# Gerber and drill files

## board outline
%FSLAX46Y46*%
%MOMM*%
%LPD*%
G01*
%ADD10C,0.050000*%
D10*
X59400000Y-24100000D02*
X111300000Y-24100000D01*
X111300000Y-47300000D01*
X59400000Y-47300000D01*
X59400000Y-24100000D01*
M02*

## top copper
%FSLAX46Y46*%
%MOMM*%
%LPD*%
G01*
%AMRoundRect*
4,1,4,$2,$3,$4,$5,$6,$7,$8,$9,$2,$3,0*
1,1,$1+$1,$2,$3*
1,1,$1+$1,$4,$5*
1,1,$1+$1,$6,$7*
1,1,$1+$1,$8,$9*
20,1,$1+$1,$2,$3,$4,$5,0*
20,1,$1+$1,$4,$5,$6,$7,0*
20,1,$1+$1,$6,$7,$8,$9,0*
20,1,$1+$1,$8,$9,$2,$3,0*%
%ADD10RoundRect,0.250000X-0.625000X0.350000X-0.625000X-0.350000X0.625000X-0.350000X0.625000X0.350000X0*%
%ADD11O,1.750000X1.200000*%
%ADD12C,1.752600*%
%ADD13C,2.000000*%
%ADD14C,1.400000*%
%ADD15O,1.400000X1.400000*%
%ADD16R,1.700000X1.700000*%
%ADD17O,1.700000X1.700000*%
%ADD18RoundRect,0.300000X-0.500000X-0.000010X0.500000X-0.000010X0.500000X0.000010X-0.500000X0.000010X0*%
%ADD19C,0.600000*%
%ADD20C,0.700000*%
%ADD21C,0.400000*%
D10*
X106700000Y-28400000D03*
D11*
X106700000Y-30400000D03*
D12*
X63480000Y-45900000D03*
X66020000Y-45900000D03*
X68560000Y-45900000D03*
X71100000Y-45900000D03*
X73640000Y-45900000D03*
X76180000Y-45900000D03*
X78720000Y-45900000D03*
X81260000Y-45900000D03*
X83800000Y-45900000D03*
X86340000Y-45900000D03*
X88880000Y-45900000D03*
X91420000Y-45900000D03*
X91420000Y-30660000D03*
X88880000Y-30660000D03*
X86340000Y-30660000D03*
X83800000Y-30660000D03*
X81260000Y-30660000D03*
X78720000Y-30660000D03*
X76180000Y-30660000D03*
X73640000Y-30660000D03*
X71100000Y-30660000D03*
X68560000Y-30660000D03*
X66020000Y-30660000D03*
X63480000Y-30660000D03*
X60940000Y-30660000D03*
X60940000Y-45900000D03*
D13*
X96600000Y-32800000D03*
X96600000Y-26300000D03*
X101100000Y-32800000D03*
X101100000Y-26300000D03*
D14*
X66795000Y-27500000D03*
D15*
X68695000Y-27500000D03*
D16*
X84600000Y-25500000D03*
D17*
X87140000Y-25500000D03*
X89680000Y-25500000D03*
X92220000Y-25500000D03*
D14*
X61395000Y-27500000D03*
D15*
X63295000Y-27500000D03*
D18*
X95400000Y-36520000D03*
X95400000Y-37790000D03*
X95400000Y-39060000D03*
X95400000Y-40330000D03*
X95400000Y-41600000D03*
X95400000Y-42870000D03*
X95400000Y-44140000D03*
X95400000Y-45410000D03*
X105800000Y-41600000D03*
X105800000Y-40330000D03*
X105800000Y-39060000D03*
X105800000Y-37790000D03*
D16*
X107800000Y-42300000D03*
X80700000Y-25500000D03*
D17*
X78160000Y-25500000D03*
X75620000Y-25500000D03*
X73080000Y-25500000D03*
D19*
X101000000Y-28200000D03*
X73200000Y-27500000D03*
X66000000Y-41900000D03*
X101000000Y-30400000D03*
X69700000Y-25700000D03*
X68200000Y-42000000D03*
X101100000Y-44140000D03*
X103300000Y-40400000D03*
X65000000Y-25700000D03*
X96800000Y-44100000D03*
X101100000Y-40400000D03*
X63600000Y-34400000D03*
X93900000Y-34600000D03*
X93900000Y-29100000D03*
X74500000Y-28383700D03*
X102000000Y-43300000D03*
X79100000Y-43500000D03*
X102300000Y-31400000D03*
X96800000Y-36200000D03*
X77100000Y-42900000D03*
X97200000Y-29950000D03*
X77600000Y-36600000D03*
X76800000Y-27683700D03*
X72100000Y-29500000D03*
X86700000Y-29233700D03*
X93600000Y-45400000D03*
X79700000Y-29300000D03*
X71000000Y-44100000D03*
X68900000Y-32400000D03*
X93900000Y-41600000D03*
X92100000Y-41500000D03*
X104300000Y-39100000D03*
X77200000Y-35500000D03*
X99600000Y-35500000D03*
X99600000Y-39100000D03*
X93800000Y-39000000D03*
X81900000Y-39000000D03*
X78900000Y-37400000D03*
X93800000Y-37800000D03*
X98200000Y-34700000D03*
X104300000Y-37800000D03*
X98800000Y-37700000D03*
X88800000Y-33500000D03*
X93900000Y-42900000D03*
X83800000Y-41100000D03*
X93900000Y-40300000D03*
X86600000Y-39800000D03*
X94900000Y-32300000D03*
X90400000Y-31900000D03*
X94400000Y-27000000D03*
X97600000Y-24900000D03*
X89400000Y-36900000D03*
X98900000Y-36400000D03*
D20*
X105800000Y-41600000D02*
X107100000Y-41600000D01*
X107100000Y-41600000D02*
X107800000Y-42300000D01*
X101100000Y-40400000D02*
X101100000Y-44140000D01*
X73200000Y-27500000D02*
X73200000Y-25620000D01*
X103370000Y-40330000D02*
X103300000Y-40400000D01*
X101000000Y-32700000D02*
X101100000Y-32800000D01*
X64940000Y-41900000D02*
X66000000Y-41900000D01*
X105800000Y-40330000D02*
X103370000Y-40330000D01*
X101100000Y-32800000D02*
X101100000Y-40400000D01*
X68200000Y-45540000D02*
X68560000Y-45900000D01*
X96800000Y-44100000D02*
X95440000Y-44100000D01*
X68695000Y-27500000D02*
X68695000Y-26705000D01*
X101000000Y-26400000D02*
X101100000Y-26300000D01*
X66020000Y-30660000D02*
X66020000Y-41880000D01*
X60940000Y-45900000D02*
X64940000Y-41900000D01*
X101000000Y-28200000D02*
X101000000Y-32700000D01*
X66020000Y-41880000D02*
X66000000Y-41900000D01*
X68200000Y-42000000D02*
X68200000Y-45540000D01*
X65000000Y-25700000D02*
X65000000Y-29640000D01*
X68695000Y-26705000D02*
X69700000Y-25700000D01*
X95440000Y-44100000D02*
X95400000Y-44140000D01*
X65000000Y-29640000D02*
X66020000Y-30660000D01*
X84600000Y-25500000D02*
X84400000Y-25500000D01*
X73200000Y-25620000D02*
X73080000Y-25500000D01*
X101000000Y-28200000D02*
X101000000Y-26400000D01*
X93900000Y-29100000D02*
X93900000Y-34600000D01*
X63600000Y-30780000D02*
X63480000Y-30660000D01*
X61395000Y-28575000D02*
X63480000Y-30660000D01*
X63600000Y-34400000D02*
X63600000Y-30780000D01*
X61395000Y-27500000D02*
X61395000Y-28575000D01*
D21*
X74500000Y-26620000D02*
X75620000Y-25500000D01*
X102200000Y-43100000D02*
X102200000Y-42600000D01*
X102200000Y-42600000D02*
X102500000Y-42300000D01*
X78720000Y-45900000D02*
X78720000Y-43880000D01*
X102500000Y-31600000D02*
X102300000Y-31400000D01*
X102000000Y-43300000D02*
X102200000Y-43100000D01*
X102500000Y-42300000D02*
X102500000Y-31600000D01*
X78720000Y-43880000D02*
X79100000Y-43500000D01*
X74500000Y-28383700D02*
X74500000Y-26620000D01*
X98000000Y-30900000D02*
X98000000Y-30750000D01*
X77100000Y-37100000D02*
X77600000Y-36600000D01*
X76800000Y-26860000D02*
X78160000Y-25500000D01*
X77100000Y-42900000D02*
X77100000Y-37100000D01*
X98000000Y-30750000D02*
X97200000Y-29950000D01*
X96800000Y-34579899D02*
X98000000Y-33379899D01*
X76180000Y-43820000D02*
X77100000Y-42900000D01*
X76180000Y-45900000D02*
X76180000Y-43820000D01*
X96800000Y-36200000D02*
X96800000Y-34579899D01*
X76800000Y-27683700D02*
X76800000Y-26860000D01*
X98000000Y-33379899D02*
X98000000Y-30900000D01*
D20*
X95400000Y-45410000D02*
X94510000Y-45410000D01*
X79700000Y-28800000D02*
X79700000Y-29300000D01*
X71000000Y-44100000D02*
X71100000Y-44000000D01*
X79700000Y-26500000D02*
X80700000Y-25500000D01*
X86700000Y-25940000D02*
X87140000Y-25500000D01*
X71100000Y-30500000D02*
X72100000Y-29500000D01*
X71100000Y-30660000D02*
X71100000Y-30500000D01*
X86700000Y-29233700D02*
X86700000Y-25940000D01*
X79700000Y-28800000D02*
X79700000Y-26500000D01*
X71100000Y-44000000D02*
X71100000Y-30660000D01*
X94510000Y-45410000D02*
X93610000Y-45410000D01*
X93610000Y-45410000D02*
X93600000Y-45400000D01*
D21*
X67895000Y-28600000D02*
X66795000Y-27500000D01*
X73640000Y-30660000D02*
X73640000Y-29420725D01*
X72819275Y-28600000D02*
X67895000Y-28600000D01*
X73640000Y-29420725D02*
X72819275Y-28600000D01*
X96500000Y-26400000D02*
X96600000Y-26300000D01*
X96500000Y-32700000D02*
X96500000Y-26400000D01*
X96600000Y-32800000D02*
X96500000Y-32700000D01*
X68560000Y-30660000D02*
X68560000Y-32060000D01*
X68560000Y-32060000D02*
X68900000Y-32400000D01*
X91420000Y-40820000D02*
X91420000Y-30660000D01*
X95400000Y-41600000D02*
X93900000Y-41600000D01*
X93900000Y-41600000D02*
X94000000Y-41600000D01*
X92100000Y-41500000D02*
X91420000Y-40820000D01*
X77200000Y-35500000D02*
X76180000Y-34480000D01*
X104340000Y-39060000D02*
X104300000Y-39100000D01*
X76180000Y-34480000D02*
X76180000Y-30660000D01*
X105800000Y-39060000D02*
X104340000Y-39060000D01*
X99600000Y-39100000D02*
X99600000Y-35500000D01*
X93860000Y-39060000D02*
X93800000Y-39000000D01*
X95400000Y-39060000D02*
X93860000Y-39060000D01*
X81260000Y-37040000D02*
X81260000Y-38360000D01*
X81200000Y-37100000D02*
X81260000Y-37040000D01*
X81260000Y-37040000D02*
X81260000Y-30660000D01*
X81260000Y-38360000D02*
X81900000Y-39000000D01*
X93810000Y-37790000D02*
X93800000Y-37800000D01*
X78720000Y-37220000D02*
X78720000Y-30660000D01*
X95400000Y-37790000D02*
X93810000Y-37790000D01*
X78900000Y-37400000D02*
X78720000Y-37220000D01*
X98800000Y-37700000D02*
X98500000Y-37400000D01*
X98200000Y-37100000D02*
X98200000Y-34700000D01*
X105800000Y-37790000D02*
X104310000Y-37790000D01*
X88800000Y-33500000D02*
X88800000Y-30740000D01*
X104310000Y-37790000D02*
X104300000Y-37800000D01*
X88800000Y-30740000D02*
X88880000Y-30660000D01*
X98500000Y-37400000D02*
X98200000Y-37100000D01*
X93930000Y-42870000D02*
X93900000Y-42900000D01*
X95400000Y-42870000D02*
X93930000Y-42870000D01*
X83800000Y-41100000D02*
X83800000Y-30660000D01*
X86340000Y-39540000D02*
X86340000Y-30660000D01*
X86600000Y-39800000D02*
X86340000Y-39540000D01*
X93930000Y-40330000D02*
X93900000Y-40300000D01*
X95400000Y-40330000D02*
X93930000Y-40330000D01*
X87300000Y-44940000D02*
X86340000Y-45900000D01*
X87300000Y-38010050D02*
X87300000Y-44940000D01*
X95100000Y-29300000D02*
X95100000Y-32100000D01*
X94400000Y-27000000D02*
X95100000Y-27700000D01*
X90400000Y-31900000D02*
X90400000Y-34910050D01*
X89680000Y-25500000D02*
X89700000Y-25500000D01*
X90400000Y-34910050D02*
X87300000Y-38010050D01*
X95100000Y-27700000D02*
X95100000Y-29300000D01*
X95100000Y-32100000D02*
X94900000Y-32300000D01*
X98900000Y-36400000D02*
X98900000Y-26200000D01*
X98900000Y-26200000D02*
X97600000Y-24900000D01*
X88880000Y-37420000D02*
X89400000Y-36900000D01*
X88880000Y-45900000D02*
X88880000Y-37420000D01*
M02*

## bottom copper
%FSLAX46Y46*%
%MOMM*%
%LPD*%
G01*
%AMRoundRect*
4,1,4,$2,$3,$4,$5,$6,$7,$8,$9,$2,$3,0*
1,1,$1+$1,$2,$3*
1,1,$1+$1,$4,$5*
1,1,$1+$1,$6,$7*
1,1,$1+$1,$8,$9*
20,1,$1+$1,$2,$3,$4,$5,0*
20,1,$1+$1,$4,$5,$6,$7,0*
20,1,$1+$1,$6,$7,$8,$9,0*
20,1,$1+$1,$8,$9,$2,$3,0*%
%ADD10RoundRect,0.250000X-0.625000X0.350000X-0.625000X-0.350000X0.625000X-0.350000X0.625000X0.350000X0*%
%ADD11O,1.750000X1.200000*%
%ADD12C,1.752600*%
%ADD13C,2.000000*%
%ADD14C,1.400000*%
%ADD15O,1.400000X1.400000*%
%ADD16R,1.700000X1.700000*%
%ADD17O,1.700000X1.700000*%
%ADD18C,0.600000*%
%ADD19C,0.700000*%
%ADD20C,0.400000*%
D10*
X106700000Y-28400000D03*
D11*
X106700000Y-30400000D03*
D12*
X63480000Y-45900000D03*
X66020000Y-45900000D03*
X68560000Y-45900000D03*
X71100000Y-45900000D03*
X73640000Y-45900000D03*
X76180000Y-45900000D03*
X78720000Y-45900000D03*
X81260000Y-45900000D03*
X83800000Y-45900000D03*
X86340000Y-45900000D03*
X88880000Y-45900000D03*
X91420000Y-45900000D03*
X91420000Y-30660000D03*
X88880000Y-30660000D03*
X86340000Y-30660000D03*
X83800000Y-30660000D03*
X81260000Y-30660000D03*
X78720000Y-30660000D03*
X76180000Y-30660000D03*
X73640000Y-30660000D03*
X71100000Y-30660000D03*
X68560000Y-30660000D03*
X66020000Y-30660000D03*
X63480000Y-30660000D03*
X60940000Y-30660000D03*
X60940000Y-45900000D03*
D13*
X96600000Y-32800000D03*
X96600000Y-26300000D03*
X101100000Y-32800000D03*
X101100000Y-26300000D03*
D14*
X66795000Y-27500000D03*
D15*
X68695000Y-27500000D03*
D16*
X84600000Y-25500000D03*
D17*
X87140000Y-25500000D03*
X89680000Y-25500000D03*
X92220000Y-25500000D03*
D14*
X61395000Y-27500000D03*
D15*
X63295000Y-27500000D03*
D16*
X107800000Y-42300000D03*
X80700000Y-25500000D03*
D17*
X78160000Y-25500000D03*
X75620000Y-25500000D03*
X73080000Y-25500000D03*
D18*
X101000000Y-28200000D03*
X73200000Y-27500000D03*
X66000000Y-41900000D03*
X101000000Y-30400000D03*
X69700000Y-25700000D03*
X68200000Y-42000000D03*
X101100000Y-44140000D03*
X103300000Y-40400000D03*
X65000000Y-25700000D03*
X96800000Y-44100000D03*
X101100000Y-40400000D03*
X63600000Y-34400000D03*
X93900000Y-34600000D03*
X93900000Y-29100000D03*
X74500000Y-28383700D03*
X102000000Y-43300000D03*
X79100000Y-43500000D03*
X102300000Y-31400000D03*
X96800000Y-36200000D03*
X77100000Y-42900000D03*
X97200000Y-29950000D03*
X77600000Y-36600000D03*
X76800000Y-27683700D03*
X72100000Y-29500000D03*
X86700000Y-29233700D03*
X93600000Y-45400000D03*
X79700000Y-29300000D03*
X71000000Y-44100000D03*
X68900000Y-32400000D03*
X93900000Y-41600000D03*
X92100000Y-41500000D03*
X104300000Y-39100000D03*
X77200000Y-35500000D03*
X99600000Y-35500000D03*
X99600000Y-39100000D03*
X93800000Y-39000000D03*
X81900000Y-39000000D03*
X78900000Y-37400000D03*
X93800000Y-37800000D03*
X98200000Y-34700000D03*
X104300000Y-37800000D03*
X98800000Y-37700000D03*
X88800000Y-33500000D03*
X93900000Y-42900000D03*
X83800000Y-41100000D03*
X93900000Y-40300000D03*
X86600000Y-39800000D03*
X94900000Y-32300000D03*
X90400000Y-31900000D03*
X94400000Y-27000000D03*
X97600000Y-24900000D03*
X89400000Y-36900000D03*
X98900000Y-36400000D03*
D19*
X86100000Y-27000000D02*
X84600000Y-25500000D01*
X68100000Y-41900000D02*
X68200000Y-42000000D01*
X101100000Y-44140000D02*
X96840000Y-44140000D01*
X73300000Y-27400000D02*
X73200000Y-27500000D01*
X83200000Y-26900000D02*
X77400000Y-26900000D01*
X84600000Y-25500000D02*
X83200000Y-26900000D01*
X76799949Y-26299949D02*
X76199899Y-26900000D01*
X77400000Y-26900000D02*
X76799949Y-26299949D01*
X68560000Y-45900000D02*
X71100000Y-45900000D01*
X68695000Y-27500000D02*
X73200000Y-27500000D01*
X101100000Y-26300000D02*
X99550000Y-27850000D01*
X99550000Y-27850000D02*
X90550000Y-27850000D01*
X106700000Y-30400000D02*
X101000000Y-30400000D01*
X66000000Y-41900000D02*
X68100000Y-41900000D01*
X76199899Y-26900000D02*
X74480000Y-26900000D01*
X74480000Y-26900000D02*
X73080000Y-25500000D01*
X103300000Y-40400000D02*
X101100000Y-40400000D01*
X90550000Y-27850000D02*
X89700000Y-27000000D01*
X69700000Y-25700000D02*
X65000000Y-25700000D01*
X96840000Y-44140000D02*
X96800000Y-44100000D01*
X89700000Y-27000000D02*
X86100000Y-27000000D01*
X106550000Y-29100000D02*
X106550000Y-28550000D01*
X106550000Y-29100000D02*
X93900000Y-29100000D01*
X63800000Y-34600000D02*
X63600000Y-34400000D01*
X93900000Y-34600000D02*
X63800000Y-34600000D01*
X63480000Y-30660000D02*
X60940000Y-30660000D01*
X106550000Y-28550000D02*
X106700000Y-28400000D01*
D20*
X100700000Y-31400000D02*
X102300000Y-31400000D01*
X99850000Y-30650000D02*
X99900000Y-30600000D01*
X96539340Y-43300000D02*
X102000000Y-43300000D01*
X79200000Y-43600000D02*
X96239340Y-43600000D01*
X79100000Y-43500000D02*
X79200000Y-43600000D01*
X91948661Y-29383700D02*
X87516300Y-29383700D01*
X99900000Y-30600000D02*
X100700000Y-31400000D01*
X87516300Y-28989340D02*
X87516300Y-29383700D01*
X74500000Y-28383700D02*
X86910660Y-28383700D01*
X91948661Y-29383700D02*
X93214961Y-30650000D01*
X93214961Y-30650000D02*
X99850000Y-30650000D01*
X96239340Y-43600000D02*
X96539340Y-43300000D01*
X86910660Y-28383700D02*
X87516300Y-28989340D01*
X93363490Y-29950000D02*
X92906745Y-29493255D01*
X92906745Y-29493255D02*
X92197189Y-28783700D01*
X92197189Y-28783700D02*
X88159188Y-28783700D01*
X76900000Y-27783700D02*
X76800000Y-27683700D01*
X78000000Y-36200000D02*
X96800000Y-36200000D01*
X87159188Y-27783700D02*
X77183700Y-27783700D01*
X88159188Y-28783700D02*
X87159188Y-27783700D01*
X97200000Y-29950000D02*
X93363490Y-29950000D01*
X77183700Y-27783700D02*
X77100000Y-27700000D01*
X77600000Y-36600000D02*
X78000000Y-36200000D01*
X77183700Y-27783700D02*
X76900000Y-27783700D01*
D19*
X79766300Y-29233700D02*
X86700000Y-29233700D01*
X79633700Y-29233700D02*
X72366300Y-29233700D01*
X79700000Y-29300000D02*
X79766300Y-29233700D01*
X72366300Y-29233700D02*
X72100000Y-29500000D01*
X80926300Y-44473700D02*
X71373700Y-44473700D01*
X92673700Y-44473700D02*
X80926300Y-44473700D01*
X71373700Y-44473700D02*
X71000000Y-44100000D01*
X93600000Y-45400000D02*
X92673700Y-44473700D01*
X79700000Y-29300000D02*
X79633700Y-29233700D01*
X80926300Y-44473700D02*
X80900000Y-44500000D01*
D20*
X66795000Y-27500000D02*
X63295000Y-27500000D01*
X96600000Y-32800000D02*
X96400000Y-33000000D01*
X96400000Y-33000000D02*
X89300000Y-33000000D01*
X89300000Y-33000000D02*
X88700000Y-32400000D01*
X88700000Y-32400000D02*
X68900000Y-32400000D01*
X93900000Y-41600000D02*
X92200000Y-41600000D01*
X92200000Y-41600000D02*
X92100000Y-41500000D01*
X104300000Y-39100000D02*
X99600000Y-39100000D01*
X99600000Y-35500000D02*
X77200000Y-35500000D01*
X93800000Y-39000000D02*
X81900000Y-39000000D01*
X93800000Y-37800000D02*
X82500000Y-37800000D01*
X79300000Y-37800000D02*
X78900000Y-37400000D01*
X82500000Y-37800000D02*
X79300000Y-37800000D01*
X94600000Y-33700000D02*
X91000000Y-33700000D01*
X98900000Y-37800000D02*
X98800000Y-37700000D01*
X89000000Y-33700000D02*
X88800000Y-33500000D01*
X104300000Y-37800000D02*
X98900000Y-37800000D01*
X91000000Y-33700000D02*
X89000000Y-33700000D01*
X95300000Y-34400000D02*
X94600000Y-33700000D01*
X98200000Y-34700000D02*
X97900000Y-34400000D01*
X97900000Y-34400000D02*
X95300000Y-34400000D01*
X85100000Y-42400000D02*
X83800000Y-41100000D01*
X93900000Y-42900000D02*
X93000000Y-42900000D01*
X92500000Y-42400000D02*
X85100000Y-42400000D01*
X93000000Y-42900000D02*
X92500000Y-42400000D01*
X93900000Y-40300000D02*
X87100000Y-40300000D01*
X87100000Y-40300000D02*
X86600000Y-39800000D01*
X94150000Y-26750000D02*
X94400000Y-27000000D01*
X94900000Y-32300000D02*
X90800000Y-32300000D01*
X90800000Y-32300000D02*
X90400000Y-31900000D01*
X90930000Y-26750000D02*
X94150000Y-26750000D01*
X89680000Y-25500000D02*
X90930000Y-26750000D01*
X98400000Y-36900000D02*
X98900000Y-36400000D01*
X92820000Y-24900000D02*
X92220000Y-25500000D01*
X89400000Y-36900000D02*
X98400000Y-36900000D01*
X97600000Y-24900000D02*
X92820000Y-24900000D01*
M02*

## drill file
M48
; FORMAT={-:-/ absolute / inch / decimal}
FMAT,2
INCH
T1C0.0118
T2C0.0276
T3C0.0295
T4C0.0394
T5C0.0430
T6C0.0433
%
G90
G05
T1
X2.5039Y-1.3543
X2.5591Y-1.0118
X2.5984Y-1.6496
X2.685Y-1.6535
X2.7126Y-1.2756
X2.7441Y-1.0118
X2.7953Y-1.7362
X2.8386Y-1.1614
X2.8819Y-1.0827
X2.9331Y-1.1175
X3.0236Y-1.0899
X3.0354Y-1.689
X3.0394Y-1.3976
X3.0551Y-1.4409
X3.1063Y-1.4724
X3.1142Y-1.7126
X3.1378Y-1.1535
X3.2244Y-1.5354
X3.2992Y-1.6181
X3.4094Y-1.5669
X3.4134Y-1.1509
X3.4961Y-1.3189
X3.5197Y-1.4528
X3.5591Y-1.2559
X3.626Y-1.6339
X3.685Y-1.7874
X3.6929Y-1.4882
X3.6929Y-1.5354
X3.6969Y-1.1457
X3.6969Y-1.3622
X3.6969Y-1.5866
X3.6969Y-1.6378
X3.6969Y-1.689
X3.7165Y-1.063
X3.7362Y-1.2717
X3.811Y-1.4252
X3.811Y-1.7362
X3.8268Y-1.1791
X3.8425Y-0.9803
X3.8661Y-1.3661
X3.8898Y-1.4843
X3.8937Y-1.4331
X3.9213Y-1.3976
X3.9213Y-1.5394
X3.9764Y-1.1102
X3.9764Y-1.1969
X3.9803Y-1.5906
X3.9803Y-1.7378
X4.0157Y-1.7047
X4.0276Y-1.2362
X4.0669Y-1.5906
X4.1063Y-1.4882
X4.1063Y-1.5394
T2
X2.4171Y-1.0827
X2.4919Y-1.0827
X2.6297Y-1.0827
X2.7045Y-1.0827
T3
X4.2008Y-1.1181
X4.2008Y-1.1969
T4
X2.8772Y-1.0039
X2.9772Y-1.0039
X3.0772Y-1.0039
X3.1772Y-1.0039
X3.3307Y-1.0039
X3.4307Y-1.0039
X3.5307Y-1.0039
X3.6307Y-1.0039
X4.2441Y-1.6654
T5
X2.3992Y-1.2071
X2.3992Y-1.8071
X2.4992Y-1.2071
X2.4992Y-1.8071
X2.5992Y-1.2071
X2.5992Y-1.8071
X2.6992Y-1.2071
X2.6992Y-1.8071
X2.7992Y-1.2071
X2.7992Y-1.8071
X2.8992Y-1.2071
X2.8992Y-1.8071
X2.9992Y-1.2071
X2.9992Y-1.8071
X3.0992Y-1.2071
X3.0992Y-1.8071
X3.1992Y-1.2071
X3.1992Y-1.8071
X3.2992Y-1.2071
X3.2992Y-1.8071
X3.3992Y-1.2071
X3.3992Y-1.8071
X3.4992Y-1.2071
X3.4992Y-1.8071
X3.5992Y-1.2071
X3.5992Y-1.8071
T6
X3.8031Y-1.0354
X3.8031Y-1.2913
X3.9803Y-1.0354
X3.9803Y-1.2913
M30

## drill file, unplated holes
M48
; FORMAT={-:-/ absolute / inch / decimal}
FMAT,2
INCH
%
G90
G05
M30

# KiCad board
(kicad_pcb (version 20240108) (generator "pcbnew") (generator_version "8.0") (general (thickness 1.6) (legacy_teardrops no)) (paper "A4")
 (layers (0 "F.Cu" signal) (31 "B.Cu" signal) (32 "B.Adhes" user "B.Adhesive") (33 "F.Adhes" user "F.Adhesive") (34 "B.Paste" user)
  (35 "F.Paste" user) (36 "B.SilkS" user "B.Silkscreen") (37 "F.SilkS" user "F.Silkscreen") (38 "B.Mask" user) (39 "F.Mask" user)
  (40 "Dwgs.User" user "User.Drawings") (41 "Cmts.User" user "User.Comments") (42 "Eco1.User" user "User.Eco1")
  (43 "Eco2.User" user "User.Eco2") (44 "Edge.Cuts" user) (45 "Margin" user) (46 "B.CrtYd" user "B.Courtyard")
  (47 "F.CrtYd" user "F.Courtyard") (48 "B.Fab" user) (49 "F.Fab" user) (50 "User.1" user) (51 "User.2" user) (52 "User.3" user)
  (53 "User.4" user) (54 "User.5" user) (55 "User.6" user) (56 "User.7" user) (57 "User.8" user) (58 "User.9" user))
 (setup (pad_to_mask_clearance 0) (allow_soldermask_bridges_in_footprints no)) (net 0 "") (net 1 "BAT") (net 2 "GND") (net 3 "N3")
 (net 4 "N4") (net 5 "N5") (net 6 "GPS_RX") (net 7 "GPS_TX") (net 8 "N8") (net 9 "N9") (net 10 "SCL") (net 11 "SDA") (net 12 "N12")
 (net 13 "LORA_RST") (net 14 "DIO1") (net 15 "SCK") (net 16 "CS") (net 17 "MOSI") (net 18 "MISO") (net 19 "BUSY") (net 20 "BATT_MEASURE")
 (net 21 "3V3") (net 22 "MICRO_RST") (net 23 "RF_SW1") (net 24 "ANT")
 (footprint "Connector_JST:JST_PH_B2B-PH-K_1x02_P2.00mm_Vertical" (layer "F.Cu") (at 106.7 28.4 -90)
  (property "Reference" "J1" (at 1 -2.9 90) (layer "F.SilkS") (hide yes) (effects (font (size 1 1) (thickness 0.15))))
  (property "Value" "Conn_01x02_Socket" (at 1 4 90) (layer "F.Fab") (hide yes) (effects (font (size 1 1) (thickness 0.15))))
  (pad "1" thru_hole roundrect (at 0 0 270) (size 1.2 1.75) (drill 0.75) (layers "*.Cu" "*.Mask") (remove_unused_layers no)
   (roundrect_rratio 0.208333) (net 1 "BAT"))
  (pad "2" thru_hole oval (at 2 0 270) (size 1.2 1.75) (drill 0.75) (layers "*.Cu" "*.Mask") (remove_unused_layers no) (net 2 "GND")))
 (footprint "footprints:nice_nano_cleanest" (layer "F.Cu") (at 77.45 38.28)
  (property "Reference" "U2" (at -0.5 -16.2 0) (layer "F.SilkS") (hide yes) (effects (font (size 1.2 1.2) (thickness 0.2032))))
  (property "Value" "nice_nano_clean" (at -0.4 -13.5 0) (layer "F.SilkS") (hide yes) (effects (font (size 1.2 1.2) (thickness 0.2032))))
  (pad "1" thru_hole circle (at -13.97 7.62) (size 1.7526 1.7526) (drill 1.0922) (layers "*.Cu" "*.SilkS" "*.Mask")
   (remove_unused_layers no) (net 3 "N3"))
  (pad "2" thru_hole circle (at -11.43 7.62) (size 1.7526 1.7526) (drill 1.0922) (layers "*.Cu" "*.SilkS" "*.Mask")
   (remove_unused_layers no) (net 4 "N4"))
  (pad "3" thru_hole circle (at -8.89 7.62) (size 1.7526 1.7526) (drill 1.0922) (layers "*.Cu" "*.SilkS" "*.Mask") (remove_unused_layers no)
   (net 2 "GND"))
  (pad "4" thru_hole circle (at -6.35 7.62) (size 1.7526 1.7526) (drill 1.0922) (layers "*.Cu" "*.SilkS" "*.Mask") (remove_unused_layers no)
   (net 2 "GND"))
  (pad "5" thru_hole circle (at -3.81 7.62) (size 1.7526 1.7526) (drill 1.0922) (layers "*.Cu" "*.SilkS" "*.Mask") (remove_unused_layers no)
   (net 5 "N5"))
  (pad "6" thru_hole circle (at -1.27 7.62) (size 1.7526 1.7526) (drill 1.0922) (layers "*.Cu" "*.SilkS" "*.Mask") (remove_unused_layers no)
   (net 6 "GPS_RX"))
  (pad "7" thru_hole circle (at 1.27 7.62) (size 1.7526 1.7526) (drill 1.0922) (layers "*.Cu" "*.SilkS" "*.Mask") (remove_unused_layers no)
   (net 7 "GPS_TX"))
  (pad "8" thru_hole circle (at 3.81 7.62) (size 1.7526 1.7526) (drill 1.0922) (layers "*.Cu" "*.SilkS" "*.Mask") (remove_unused_layers no)
   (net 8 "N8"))
  (pad "9" thru_hole circle (at 6.35 7.62) (size 1.7526 1.7526) (drill 1.0922) (layers "*.Cu" "*.SilkS" "*.Mask") (remove_unused_layers no)
   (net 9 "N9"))
  (pad "10" thru_hole circle (at 8.89 7.62) (size 1.7526 1.7526) (drill 1.0922) (layers "*.Cu" "*.SilkS" "*.Mask") (remove_unused_layers no)
   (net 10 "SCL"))
  (pad "11" thru_hole circle (at 11.43 7.62) (size 1.7526 1.7526) (drill 1.0922) (layers "*.Cu" "*.SilkS" "*.Mask")
   (remove_unused_layers no) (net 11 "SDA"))
  (pad "12" thru_hole circle (at 13.97 7.62) (size 1.7526 1.7526) (drill 1.0922) (layers "*.Cu" "*.SilkS" "*.Mask")
   (remove_unused_layers no) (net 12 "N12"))
  (pad "13" thru_hole circle (at 13.97 -7.62) (size 1.7526 1.7526) (drill 1.0922) (layers "*.Cu" "*.SilkS" "*.Mask")
   (remove_unused_layers no) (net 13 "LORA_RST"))
  (pad "14" thru_hole circle (at 11.43 -7.62) (size 1.7526 1.7526) (drill 1.0922) (layers "*.Cu" "*.SilkS" "*.Mask")
   (remove_unused_layers no) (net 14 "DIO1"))
  (pad "15" thru_hole circle (at 8.89 -7.62) (size 1.7526 1.7526) (drill 1.0922) (layers "*.Cu" "*.SilkS" "*.Mask")
   (remove_unused_layers no) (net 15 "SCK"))
  (pad "16" thru_hole circle (at 6.35 -7.62) (size 1.7526 1.7526) (drill 1.0922) (layers "*.Cu" "*.SilkS" "*.Mask")
   (remove_unused_layers no) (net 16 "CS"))
  (pad "17" thru_hole circle (at 3.81 -7.62) (size 1.7526 1.7526) (drill 1.0922) (layers "*.Cu" "*.SilkS" "*.Mask")
   (remove_unused_layers no) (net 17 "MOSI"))
  (pad "18" thru_hole circle (at 1.27 -7.62) (size 1.7526 1.7526) (drill 1.0922) (layers "*.Cu" "*.SilkS" "*.Mask")
   (remove_unused_layers no) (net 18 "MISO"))
  (pad "19" thru_hole circle (at -1.27 -7.62) (size 1.7526 1.7526) (drill 1.0922) (layers "*.Cu" "*.SilkS" "*.Mask")
   (remove_unused_layers no) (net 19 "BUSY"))
  (pad "20" thru_hole circle (at -3.81 -7.62) (size 1.7526 1.7526) (drill 1.0922) (layers "*.Cu" "*.SilkS" "*.Mask")
   (remove_unused_layers no) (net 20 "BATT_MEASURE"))
  (pad "21" thru_hole circle (at -6.35 -7.62) (size 1.7526 1.7526) (drill 1.0922) (layers "*.Cu" "*.SilkS" "*.Mask")
   (remove_unused_layers no) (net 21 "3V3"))
  (pad "22" thru_hole circle (at -8.89 -7.62) (size 1.7526 1.7526) (drill 1.0922) (layers "*.Cu" "*.SilkS" "*.Mask")
   (remove_unused_layers no) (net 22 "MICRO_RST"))
  (pad "23" thru_hole circle (at -11.43 -7.62) (size 1.7526 1.7526) (drill 1.0922) (layers "*.Cu" "*.SilkS" "*.Mask")
   (remove_unused_layers no) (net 2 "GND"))
  (pad "24" thru_hole circle (at -13.97 -7.62) (size 1.7526 1.7526) (drill 1.0922) (layers "*.Cu" "*.SilkS" "*.Mask")
   (remove_unused_layers no) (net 1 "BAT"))
  (pad "25" thru_hole circle (at -16.51 -7.62) (size 1.7526 1.7526) (drill 1.0922) (layers "*.Cu" "*.SilkS" "*.Mask")
   (remove_unused_layers no) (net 1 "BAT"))
  (pad "26" thru_hole circle (at -16.51 7.62) (size 1.7526 1.7526) (drill 1.0922) (layers "*.Cu" "*.SilkS" "*.Mask")
   (remove_unused_layers no) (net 2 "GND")))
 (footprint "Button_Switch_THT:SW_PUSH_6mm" (layer "F.Cu") (at 96.6 32.8 90)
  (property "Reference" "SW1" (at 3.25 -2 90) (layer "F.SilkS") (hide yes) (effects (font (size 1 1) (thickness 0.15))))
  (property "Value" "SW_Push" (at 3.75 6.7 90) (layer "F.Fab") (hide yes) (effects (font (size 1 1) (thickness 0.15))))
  (pad "1" thru_hole circle (at 0 0 180) (size 2 2) (drill 1.1) (layers "*.Cu" "*.Mask") (remove_unused_layers no) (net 22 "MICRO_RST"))
  (pad "1" thru_hole circle (at 6.5 0 180) (size 2 2) (drill 1.1) (layers "*.Cu" "*.Mask") (remove_unused_layers no) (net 22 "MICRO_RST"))
  (pad "2" thru_hole circle (at 0 4.5 180) (size 2 2) (drill 1.1) (layers "*.Cu" "*.Mask") (remove_unused_layers no) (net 2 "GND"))
  (pad "2" thru_hole circle (at 6.5 4.5 180) (size 2 2) (drill 1.1) (layers "*.Cu" "*.Mask") (remove_unused_layers no) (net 2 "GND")))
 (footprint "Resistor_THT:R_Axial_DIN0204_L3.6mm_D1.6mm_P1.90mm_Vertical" (layer "F.Cu") (at 66.795 27.5)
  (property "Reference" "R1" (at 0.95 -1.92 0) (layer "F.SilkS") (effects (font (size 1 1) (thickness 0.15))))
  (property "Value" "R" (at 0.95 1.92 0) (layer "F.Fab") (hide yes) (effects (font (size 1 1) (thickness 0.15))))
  (pad "1" thru_hole circle (at 0 0) (size 1.4 1.4) (drill 0.7) (layers "*.Cu" "*.Mask") (remove_unused_layers no) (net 20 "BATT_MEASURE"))
  (pad "2" thru_hole oval (at 1.9 0) (size 1.4 1.4) (drill 0.7) (layers "*.Cu" "*.Mask") (remove_unused_layers no) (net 2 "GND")))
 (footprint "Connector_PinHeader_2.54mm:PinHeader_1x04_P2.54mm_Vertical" (layer "F.Cu") (at 84.6 25.5 90)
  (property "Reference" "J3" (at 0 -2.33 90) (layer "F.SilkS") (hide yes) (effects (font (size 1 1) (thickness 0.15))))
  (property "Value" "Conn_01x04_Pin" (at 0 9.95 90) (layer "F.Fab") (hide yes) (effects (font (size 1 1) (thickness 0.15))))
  (pad "1" thru_hole rect (at 0 0 90) (size 1.7 1.7) (drill 1) (layers "*.Cu" "*.Mask") (remove_unused_layers no) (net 2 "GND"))
  (pad "2" thru_hole oval (at 0 2.54 90) (size 1.7 1.7) (drill 1) (layers "*.Cu" "*.Mask") (remove_unused_layers no) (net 21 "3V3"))
  (pad "3" thru_hole oval (at 0 5.08 90) (size 1.7 1.7) (drill 1) (layers "*.Cu" "*.Mask") (remove_unused_layers no) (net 10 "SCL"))
  (pad "4" thru_hole oval (at 0 7.62 90) (size 1.7 1.7) (drill 1) (layers "*.Cu" "*.Mask") (remove_unused_layers no) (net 11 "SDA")))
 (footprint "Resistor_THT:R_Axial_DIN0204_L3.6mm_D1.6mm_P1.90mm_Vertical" (layer "F.Cu") (at 61.395 27.5)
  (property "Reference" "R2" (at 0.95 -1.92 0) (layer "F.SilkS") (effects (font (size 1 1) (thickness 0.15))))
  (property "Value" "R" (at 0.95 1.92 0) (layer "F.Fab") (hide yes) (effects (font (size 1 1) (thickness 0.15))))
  (pad "1" thru_hole circle (at 0 0) (size 1.4 1.4) (drill 0.7) (layers "*.Cu" "*.Mask") (remove_unused_layers no) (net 1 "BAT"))
  (pad "2" thru_hole oval (at 1.9 0) (size 1.4 1.4) (drill 0.7) (layers "*.Cu" "*.Mask") (remove_unused_layers no) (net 20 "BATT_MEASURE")))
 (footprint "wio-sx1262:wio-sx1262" (layer "F.Cu") (at 95.1 35.19 -90)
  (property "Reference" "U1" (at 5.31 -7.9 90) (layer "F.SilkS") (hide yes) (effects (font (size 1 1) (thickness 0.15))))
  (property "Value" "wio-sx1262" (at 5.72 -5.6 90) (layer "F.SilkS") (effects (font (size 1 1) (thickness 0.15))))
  (pad "1" smd roundrect (at 1.33 -0.3) (size 1.6 0.6) (layers "F.Cu" "F.Paste" "F.Mask") (roundrect_rratio 0.5) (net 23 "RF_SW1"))
  (pad "2" smd roundrect (at 2.6 -0.3) (size 1.6 0.6) (layers "F.Cu" "F.Paste" "F.Mask") (roundrect_rratio 0.5) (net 18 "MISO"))
  (pad "3" smd roundrect (at 3.87 -0.3) (size 1.6 0.6) (layers "F.Cu" "F.Paste" "F.Mask") (roundrect_rratio 0.5) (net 17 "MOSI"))
  (pad "4" smd roundrect (at 5.14 -0.3) (size 1.6 0.6) (layers "F.Cu" "F.Paste" "F.Mask") (roundrect_rratio 0.5) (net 15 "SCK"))
  (pad "5" smd roundrect (at 6.41 -0.3) (size 1.6 0.6) (layers "F.Cu" "F.Paste" "F.Mask") (roundrect_rratio 0.5) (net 13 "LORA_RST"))
  (pad "6" smd roundrect (at 7.68 -0.3) (size 1.6 0.6) (layers "F.Cu" "F.Paste" "F.Mask") (roundrect_rratio 0.5) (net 16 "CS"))
  (pad "7" smd roundrect (at 8.95 -0.3) (size 1.6 0.6) (layers "F.Cu" "F.Paste" "F.Mask") (roundrect_rratio 0.5) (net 2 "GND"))
  (pad "8" smd roundrect (at 10.22 -0.3) (size 1.6 0.6) (layers "F.Cu" "F.Paste" "F.Mask") (roundrect_rratio 0.5) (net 21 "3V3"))
  (pad "9" smd roundrect (at 6.41 -10.7) (size 1.6 0.6) (layers "F.Cu" "F.Paste" "F.Mask") (roundrect_rratio 0.5) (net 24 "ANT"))
  (pad "10" smd roundrect (at 5.14 -10.7) (size 1.6 0.6) (layers "F.Cu" "F.Paste" "F.Mask") (roundrect_rratio 0.5) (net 2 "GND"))
  (pad "11" smd roundrect (at 3.87 -10.7) (size 1.6 0.6) (layers "F.Cu" "F.Paste" "F.Mask") (roundrect_rratio 0.5) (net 19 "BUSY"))
  (pad "12" smd roundrect (at 2.6 -10.7) (size 1.6 0.6) (layers "F.Cu" "F.Paste" "F.Mask") (roundrect_rratio 0.5) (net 14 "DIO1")))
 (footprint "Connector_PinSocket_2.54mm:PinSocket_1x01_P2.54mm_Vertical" (layer "F.Cu") (at 107.8 42.3)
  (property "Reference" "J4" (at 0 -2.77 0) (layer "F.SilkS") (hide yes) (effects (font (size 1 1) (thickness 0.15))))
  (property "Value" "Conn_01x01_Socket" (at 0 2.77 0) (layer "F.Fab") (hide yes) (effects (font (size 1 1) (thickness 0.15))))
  (pad "1" thru_hole rect (at 0 0) (size 1.7 1.7) (drill 1) (layers "*.Cu" "*.Mask") (remove_unused_layers no) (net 24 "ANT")))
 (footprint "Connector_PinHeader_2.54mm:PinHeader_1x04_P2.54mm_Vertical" (layer "B.Cu") (at 80.7 25.5 90)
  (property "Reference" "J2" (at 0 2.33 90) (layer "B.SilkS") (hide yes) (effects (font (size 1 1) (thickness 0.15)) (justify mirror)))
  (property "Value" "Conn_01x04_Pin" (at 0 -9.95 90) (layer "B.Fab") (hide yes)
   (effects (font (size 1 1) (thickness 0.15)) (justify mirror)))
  (pad "1" thru_hole rect (at 0 0 90) (size 1.7 1.7) (drill 1) (layers "*.Cu" "*.Mask") (remove_unused_layers no) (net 21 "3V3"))
  (pad "2" thru_hole oval (at 0 -2.54 90) (size 1.7 1.7) (drill 1) (layers "*.Cu" "*.Mask") (remove_unused_layers no) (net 6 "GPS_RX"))
  (pad "3" thru_hole oval (at 0 -5.08 90) (size 1.7 1.7) (drill 1) (layers "*.Cu" "*.Mask") (remove_unused_layers no) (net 7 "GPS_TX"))
  (pad "4" thru_hole oval (at 0 -7.62 90) (size 1.7 1.7) (drill 1) (layers "*.Cu" "*.Mask") (remove_unused_layers no) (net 2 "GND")))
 (gr_rect (start 59.4 24.1) (end 111.3 47.3) (stroke (width 0.05) (type default)) (fill none) (layer "Edge.Cuts"))
 (segment (start 101.1 40.4) (end 101.1 44.14) (width 0.7) (layer "F.Cu") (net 2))
 (segment (start 73.2 27.5) (end 73.2 25.62) (width 0.7) (layer "F.Cu") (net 2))
 (segment (start 103.37 40.33) (end 103.3 40.4) (width 0.7) (layer "F.Cu") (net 2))
 (segment (start 101 32.7) (end 101.1 32.8) (width 0.7) (layer "F.Cu") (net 2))
 (segment (start 64.94 41.9) (end 66 41.9) (width 0.7) (layer "F.Cu") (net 2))
 (segment (start 105.8 40.33) (end 103.37 40.33) (width 0.7) (layer "F.Cu") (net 2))
 (segment (start 101.1 32.8) (end 101.1 40.4) (width 0.7) (layer "F.Cu") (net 2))
 (segment (start 68.2 45.54) (end 68.56 45.9) (width 0.7) (layer "F.Cu") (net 2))
 (segment (start 96.8 44.1) (end 95.44 44.1) (width 0.7) (layer "F.Cu") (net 2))
 (segment (start 68.695 27.5) (end 68.695 26.705) (width 0.7) (layer "F.Cu") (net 2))
 (segment (start 101 26.4) (end 101.1 26.3) (width 0.7) (layer "F.Cu") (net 2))
 (segment (start 66.02 30.66) (end 66.02 41.88) (width 0.7) (layer "F.Cu") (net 2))
 (segment (start 60.94 45.9) (end 64.94 41.9) (width 0.7) (layer "F.Cu") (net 2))
 (segment (start 101 28.2) (end 101 32.7) (width 0.7) (layer "F.Cu") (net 2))
 (segment (start 66.02 41.88) (end 66 41.9) (width 0.7) (layer "F.Cu") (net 2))
 (segment (start 68.2 42) (end 68.2 45.54) (width 0.7) (layer "F.Cu") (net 2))
 (segment (start 65 25.7) (end 65 29.64) (width 0.7) (layer "F.Cu") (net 2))
 (segment (start 68.695 26.705) (end 69.7 25.7) (width 0.7) (layer "F.Cu") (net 2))
 (segment (start 95.44 44.1) (end 95.4 44.14) (width 0.7) (layer "F.Cu") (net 2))
 (segment (start 65 29.64) (end 66.02 30.66) (width 0.7) (layer "F.Cu") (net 2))
 (segment (start 84.6 25.5) (end 84.4 25.5) (width 0.7) (layer "F.Cu") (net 2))
 (segment (start 73.2 25.62) (end 73.08 25.5) (width 0.7) (layer "F.Cu") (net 2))
 (segment (start 101 28.2) (end 101 26.4) (width 0.7) (layer "F.Cu") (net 2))
 (via (at 101 28.2) (size 0.6) (drill 0.3) (layers "F.Cu" "B.Cu") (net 2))
 (via (at 73.2 27.5) (size 0.6) (drill 0.3) (layers "F.Cu" "B.Cu") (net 2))
 (via (at 66 41.9) (size 0.6) (drill 0.3) (layers "F.Cu" "B.Cu") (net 2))
 (via (at 101 30.4) (size 0.6) (drill 0.3) (layers "F.Cu" "B.Cu") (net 2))
 (via (at 69.7 25.7) (size 0.6) (drill 0.3) (layers "F.Cu" "B.Cu") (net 2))
 (via (at 68.2 42) (size 0.6) (drill 0.3) (layers "F.Cu" "B.Cu") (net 2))
 (via (at 101.1 44.14) (size 0.6) (drill 0.3) (layers "F.Cu" "B.Cu") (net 2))
 (via (at 103.3 40.4) (size 0.6) (drill 0.3) (layers "F.Cu" "B.Cu") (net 2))
 (via (at 65 25.7) (size 0.6) (drill 0.3) (layers "F.Cu" "B.Cu") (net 2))
 (via (at 96.8 44.1) (size 0.6) (drill 0.3) (layers "F.Cu" "B.Cu") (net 2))
 (via (at 101.1 40.4) (size 0.6) (drill 0.3) (layers "F.Cu" "B.Cu") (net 2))
 (segment (start 86.1 27) (end 84.6 25.5) (width 0.7) (layer "B.Cu") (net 2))
 (segment (start 68.1 41.9) (end 68.2 42) (width 0.7) (layer "B.Cu") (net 2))
 (segment (start 101.1 44.14) (end 96.84 44.14) (width 0.7) (layer "B.Cu") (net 2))
 (segment (start 73.3 27.4) (end 73.2 27.5) (width 0.7) (layer "B.Cu") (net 2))
 (segment (start 83.2 26.9) (end 77.4 26.9) (width 0.7) (layer "B.Cu") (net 2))
 (segment (start 84.6 25.5) (end 83.2 26.9) (width 0.7) (layer "B.Cu") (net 2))
 (segment (start 76.799949 26.299949) (end 76.199899 26.9) (width 0.7) (layer "B.Cu") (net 2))
 (segment (start 77.4 26.9) (end 76.799949 26.299949) (width 0.7) (layer "B.Cu") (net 2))
 (segment (start 68.56 45.9) (end 71.1 45.9) (width 0.7) (layer "B.Cu") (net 2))
 (segment (start 68.695 27.5) (end 73.2 27.5) (width 0.7) (layer "B.Cu") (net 2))
 (segment (start 101.1 26.3) (end 99.55 27.85) (width 0.7) (layer "B.Cu") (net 2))
 (segment (start 99.55 27.85) (end 90.55 27.85) (width 0.7) (layer "B.Cu") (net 2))
 (segment (start 106.7 30.4) (end 101 30.4) (width 0.7) (layer "B.Cu") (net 2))
 (segment (start 66 41.9) (end 68.1 41.9) (width 0.7) (layer "B.Cu") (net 2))
 (segment (start 76.199899 26.9) (end 74.48 26.9) (width 0.7) (layer "B.Cu") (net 2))
 (segment (start 74.48 26.9) (end 73.08 25.5) (width 0.7) (layer "B.Cu") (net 2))
 (segment (start 103.3 40.4) (end 101.1 40.4) (width 0.7) (layer "B.Cu") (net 2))
 (segment (start 90.55 27.85) (end 89.7 27) (width 0.7) (layer "B.Cu") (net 2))
 (segment (start 69.7 25.7) (end 65 25.7) (width 0.7) (layer "B.Cu") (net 2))
 (segment (start 96.84 44.14) (end 96.8 44.1) (width 0.7) (layer "B.Cu") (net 2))
 (segment (start 89.7 27) (end 86.1 27) (width 0.7) (layer "B.Cu") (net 2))
 (segment (start 93.9 29.1) (end 93.9 34.6) (width 0.7) (layer "F.Cu") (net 1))
 (segment (start 63.6 30.78) (end 63.48 30.66) (width 0.7) (layer "F.Cu") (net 1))
 (segment (start 61.395 28.575) (end 63.48 30.66) (width 0.7) (layer "F.Cu") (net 1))
 (segment (start 63.6 34.4) (end 63.6 30.78) (width 0.7) (layer "F.Cu") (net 1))
 (segment (start 61.395 27.5) (end 61.395 28.575) (width 0.7) (layer "F.Cu") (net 1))
 (via (at 63.6 34.4) (size 0.6) (drill 0.3) (layers "F.Cu" "B.Cu") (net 1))
 (via (at 93.9 34.6) (size 0.6) (drill 0.3) (layers "F.Cu" "B.Cu") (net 1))
 (via (at 93.9 29.1) (size 0.6) (drill 0.3) (layers "F.Cu" "B.Cu") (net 1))
 (segment (start 106.55 29.1) (end 106.55 28.55) (width 0.7) (layer "B.Cu") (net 1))
 (segment (start 106.55 29.1) (end 93.9 29.1) (width 0.7) (layer "B.Cu") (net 1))
 (segment (start 63.8 34.6) (end 63.6 34.4) (width 0.7) (layer "B.Cu") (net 1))
 (segment (start 93.9 34.6) (end 63.8 34.6) (width 0.7) (layer "B.Cu") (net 1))
 (segment (start 63.48 30.66) (end 60.94 30.66) (width 0.7) (layer "B.Cu") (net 1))
 (segment (start 106.55 28.55) (end 106.7 28.4) (width 0.7) (layer "B.Cu") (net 1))
 (segment (start 74.5 26.62) (end 75.62 25.5) (width 0.4) (layer "F.Cu") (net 7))
 (segment (start 102.2 43.1) (end 102.2 42.6) (width 0.4) (layer "F.Cu") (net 7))
 (segment (start 102.2 42.6) (end 102.5 42.3) (width 0.4) (layer "F.Cu") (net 7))
 (segment (start 78.72 45.9) (end 78.72 43.88) (width 0.4) (layer "F.Cu") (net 7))
 (segment (start 102.5 31.6) (end 102.3 31.4) (width 0.4) (layer "F.Cu") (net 7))
 (segment (start 102 43.3) (end 102.2 43.1) (width 0.4) (layer "F.Cu") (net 7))
 (segment (start 102.5 42.3) (end 102.5 31.6) (width 0.4) (layer "F.Cu") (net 7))
 (segment (start 78.72 43.88) (end 79.1 43.5) (width 0.4) (layer "F.Cu") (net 7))
 (segment (start 74.5 28.3837) (end 74.5 26.62) (width 0.4) (layer "F.Cu") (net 7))
 (via (at 74.5 28.3837) (size 0.6) (drill 0.3) (layers "F.Cu" "B.Cu") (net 7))
 (via (at 102 43.3) (size 0.6) (drill 0.3) (layers "F.Cu" "B.Cu") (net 7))
 (via (at 79.1 43.5) (size 0.6) (drill 0.3) (layers "F.Cu" "B.Cu") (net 7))
 (via (at 102.3 31.4) (size 0.6) (drill 0.3) (layers "F.Cu" "B.Cu") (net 7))
 (segment (start 100.7 31.4) (end 102.3 31.4) (width 0.4) (layer "B.Cu") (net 7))
 (segment (start 99.85 30.65) (end 99.9 30.6) (width 0.4) (layer "B.Cu") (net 7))
 (segment (start 96.53934 43.3) (end 102 43.3) (width 0.4) (layer "B.Cu") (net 7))
 (segment (start 79.2 43.6) (end 96.23934 43.6) (width 0.4) (layer "B.Cu") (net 7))
 (segment (start 79.1 43.5) (end 79.2 43.6) (width 0.4) (layer "B.Cu") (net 7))
 (segment (start 91.948661 29.3837) (end 87.5163 29.3837) (width 0.4) (layer "B.Cu") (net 7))
 (segment (start 99.9 30.6) (end 100.7 31.4) (width 0.4) (layer "B.Cu") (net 7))
 (segment (start 87.5163 28.98934) (end 87.5163 29.3837) (width 0.4) (layer "B.Cu") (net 7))
 (segment (start 74.5 28.3837) (end 86.91066 28.3837) (width 0.4) (layer "B.Cu") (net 7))
 (segment (start 91.948661 29.3837) (end 93.214961 30.65) (width 0.4) (layer "B.Cu") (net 7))
 (segment (start 93.214961 30.65) (end 99.85 30.65) (width 0.4) (layer "B.Cu") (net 7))
 (segment (start 96.23934 43.6) (end 96.53934 43.3) (width 0.4) (layer "B.Cu") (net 7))
 (segment (start 86.91066 28.3837) (end 87.5163 28.98934) (width 0.4) (layer "B.Cu") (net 7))
 (segment (start 98 30.9) (end 98 30.75) (width 0.4) (layer "F.Cu") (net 6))
 (segment (start 77.1 37.1) (end 77.6 36.6) (width 0.4) (layer "F.Cu") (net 6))
 (segment (start 76.8 26.86) (end 78.16 25.5) (width 0.4) (layer "F.Cu") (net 6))
 (segment (start 77.1 42.9) (end 77.1 37.1) (width 0.4) (layer "F.Cu") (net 6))
 (segment (start 98 30.75) (end 97.2 29.95) (width 0.4) (layer "F.Cu") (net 6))
 (segment (start 96.8 34.579899) (end 98 33.379899) (width 0.4) (layer "F.Cu") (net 6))
 (segment (start 76.18 43.82) (end 77.1 42.9) (width 0.4) (layer "F.Cu") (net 6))
 (segment (start 76.18 45.9) (end 76.18 43.82) (width 0.4) (layer "F.Cu") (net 6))
 (segment (start 96.8 36.2) (end 96.8 34.579899) (width 0.4) (layer "F.Cu") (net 6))
 (segment (start 76.8 27.6837) (end 76.8 26.86) (width 0.4) (layer "F.Cu") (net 6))
 (segment (start 98 33.379899) (end 98 30.9) (width 0.4) (layer "F.Cu") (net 6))
 (via (at 96.8 36.2) (size 0.6) (drill 0.3) (layers "F.Cu" "B.Cu") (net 6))
 (via (at 77.1 42.9) (size 0.6) (drill 0.3) (layers "F.Cu" "B.Cu") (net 6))
 (via (at 97.2 29.95) (size 0.6) (drill 0.3) (layers "F.Cu" "B.Cu") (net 6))
 (via (at 77.6 36.6) (size 0.6) (drill 0.3) (layers "F.Cu" "B.Cu") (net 6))
 (via (at 76.8 27.6837) (size 0.6) (drill 0.3) (layers "F.Cu" "B.Cu") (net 6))
 (segment (start 93.36349 29.95) (end 92.906745 29.493255) (width 0.4) (layer "B.Cu") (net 6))
 (segment (start 92.906745 29.493255) (end 92.197189 28.7837) (width 0.4) (layer "B.Cu") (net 6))
 (segment (start 92.197189 28.7837) (end 88.159188 28.7837) (width 0.4) (layer "B.Cu") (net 6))
 (segment (start 76.9 27.7837) (end 76.8 27.6837) (width 0.4) (layer "B.Cu") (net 6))
 (segment (start 78 36.2) (end 96.8 36.2) (width 0.4) (layer "B.Cu") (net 6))
 (segment (start 87.159188 27.7837) (end 77.1837 27.7837) (width 0.4) (layer "B.Cu") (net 6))
 (segment (start 88.159188 28.7837) (end 87.159188 27.7837) (width 0.4) (layer "B.Cu") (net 6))
 (segment (start 97.2 29.95) (end 93.36349 29.95) (width 0.4) (layer "B.Cu") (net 6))
 (segment (start 77.1837 27.7837) (end 77.1 27.7) (width 0.4) (layer "B.Cu") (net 6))
 (segment (start 77.6 36.6) (end 78 36.2) (width 0.4) (layer "B.Cu") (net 6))
 (segment (start 77.1837 27.7837) (end 76.9 27.7837) (width 0.4) (layer "B.Cu") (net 6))
 (segment (start 95.4 45.41) (end 94.51 45.41) (width 0.7) (layer "F.Cu") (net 21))
 (segment (start 79.7 28.8) (end 79.7 29.3) (width 0.7) (layer "F.Cu") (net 21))
 (segment (start 71 44.1) (end 71.1 44) (width 0.7) (layer "F.Cu") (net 21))
 (segment (start 79.7 26.5) (end 80.7 25.5) (width 0.7) (layer "F.Cu") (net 21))
 (segment (start 86.7 25.94) (end 87.14 25.5) (width 0.7) (layer "F.Cu") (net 21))
 (segment (start 71.1 30.5) (end 72.1 29.5) (width 0.7) (layer "F.Cu") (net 21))
 (segment (start 71.1 30.66) (end 71.1 30.5) (width 0.7) (layer "F.Cu") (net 21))
 (segment (start 86.7 29.2337) (end 86.7 25.94) (width 0.7) (layer "F.Cu") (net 21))
 (segment (start 79.7 28.8) (end 79.7 26.5) (width 0.7) (layer "F.Cu") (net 21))
 (segment (start 71.1 44) (end 71.1 30.66) (width 0.7) (layer "F.Cu") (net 21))
 (segment (start 94.51 45.41) (end 93.61 45.41) (width 0.7) (layer "F.Cu") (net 21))
 (segment (start 93.61 45.41) (end 93.6 45.4) (width 0.7) (layer "F.Cu") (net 21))
 (via (at 72.1 29.5) (size 0.6) (drill 0.3) (layers "F.Cu" "B.Cu") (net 21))
 (via (at 86.7 29.2337) (size 0.6) (drill 0.3) (layers "F.Cu" "B.Cu") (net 21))
 (via (at 93.6 45.4) (size 0.6) (drill 0.3) (layers "F.Cu" "B.Cu") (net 21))
 (via (at 79.7 29.3) (size 0.6) (drill 0.3) (layers "F.Cu" "B.Cu") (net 21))
 (via (at 71 44.1) (size 0.6) (drill 0.3) (layers "F.Cu" "B.Cu") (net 21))
 (segment (start 79.7663 29.2337) (end 86.7 29.2337) (width 0.7) (layer "B.Cu") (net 21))
 (segment (start 79.6337 29.2337) (end 72.3663 29.2337) (width 0.7) (layer "B.Cu") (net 21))
 (segment (start 79.7 29.3) (end 79.7663 29.2337) (width 0.7) (layer "B.Cu") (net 21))
 (segment (start 72.3663 29.2337) (end 72.1 29.5) (width 0.7) (layer "B.Cu") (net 21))
 (segment (start 80.9263 44.4737) (end 71.3737 44.4737) (width 0.7) (layer "B.Cu") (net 21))
 (segment (start 92.6737 44.4737) (end 80.9263 44.4737) (width 0.7) (layer "B.Cu") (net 21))
 (segment (start 71.3737 44.4737) (end 71 44.1) (width 0.7) (layer "B.Cu") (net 21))
 (segment (start 93.6 45.4) (end 92.6737 44.4737) (width 0.7) (layer "B.Cu") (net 21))
 (segment (start 79.7 29.3) (end 79.6337 29.2337) (width 0.7) (layer "B.Cu") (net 21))
 (segment (start 80.9263 44.4737) (end 80.9 44.5) (width 0.7) (layer "B.Cu") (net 21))
 (segment (start 67.895 28.6) (end 66.795 27.5) (width 0.4) (layer "F.Cu") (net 20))
 (segment (start 73.64 30.66) (end 73.64 29.420725) (width 0.4) (layer "F.Cu") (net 20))
 (segment (start 72.819275 28.6) (end 67.895 28.6) (width 0.4) (layer "F.Cu") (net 20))
 (segment (start 73.64 29.420725) (end 72.819275 28.6) (width 0.4) (layer "F.Cu") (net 20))
 (segment (start 66.795 27.5) (end 63.295 27.5) (width 0.4) (layer "B.Cu") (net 20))
 (segment (start 96.5 26.4) (end 96.6 26.3) (width 0.4) (layer "F.Cu") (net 22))
 (segment (start 96.5 32.7) (end 96.5 26.4) (width 0.4) (layer "F.Cu") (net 22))
 (segment (start 96.6 32.8) (end 96.5 32.7) (width 0.4) (layer "F.Cu") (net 22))
 (segment (start 68.56 30.66) (end 68.56 32.06) (width 0.4) (layer "F.Cu") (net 22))
 (segment (start 68.56 32.06) (end 68.9 32.4) (width 0.4) (layer "F.Cu") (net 22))
 (via (at 68.9 32.4) (size 0.6) (drill 0.3) (layers "F.Cu" "B.Cu") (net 22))
 (segment (start 96.6 32.8) (end 96.4 33) (width 0.4) (layer "B.Cu") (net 22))
 (segment (start 96.4 33) (end 89.3 33) (width 0.4) (layer "B.Cu") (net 22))
 (segment (start 89.3 33) (end 88.7 32.4) (width 0.4) (layer "B.Cu") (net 22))
 (segment (start 88.7 32.4) (end 68.9 32.4) (width 0.4) (layer "B.Cu") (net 22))
 (segment (start 91.42 40.82) (end 91.42 30.66) (width 0.4) (layer "F.Cu") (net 13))
 (segment (start 95.4 41.6) (end 93.9 41.6) (width 0.4) (layer "F.Cu") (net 13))
 (segment (start 93.9 41.6) (end 94 41.6) (width 0.4) (layer "F.Cu") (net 13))
 (segment (start 92.1 41.5) (end 91.42 40.82) (width 0.4) (layer "F.Cu") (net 13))
 (via (at 93.9 41.6) (size 0.6) (drill 0.3) (layers "F.Cu" "B.Cu") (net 13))
 (via (at 92.1 41.5) (size 0.6) (drill 0.3) (layers "F.Cu" "B.Cu") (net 13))
 (segment (start 93.9 41.6) (end 92.2 41.6) (width 0.4) (layer "B.Cu") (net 13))
 (segment (start 92.2 41.6) (end 92.1 41.5) (width 0.4) (layer "B.Cu") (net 13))
 (segment (start 77.2 35.5) (end 76.18 34.48) (width 0.4) (layer "F.Cu") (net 19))
 (segment (start 104.34 39.06) (end 104.3 39.1) (width 0.4) (layer "F.Cu") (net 19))
 (segment (start 76.18 34.48) (end 76.18 30.66) (width 0.4) (layer "F.Cu") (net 19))
 (segment (start 105.8 39.06) (end 104.34 39.06) (width 0.4) (layer "F.Cu") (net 19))
 (segment (start 99.6 39.1) (end 99.6 35.5) (width 0.4) (layer "F.Cu") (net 19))
 (via (at 104.3 39.1) (size 0.6) (drill 0.3) (layers "F.Cu" "B.Cu") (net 19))
 (via (at 77.2 35.5) (size 0.6) (drill 0.3) (layers "F.Cu" "B.Cu") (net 19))
 (via (at 99.6 35.5) (size 0.6) (drill 0.3) (layers "F.Cu" "B.Cu") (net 19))
 (via (at 99.6 39.1) (size 0.6) (drill 0.3) (layers "F.Cu" "B.Cu") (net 19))
 (segment (start 104.3 39.1) (end 99.6 39.1) (width 0.4) (layer "B.Cu") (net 19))
 (segment (start 99.6 35.5) (end 77.2 35.5) (width 0.4) (layer "B.Cu") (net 19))
 (segment (start 107.1 41.6) (end 107.8 42.3) (width 0.7) (layer "F.Cu") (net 24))
 (segment (start 105.8 41.6) (end 107.1 41.6) (width 0.7) (layer "F.Cu") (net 24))
 (segment (start 93.86 39.06) (end 93.8 39) (width 0.4) (layer "F.Cu") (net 17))
 (segment (start 95.4 39.06) (end 93.86 39.06) (width 0.4) (layer "F.Cu") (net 17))
 (segment (start 81.26 37.04) (end 81.26 38.36) (width 0.4) (layer "F.Cu") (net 17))
 (segment (start 81.2 37.1) (end 81.26 37.04) (width 0.4) (layer "F.Cu") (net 17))
 (segment (start 81.26 37.04) (end 81.26 30.66) (width 0.4) (layer "F.Cu") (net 17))
 (segment (start 81.26 38.36) (end 81.9 39) (width 0.4) (layer "F.Cu") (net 17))
 (via (at 93.8 39) (size 0.6) (drill 0.3) (layers "F.Cu" "B.Cu") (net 17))
 (via (at 81.9 39) (size 0.6) (drill 0.3) (layers "F.Cu" "B.Cu") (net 17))
 (segment (start 93.8 39) (end 81.9 39) (width 0.4) (layer "B.Cu") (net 17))
 (segment (start 93.81 37.79) (end 93.8 37.8) (width 0.4) (layer "F.Cu") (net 18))
 (segment (start 78.72 37.22) (end 78.72 30.66) (width 0.4) (layer "F.Cu") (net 18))
 (segment (start 95.4 37.79) (end 93.81 37.79) (width 0.4) (layer "F.Cu") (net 18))
 (segment (start 78.9 37.4) (end 78.72 37.22) (width 0.4) (layer "F.Cu") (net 18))
 (via (at 78.9 37.4) (size 0.6) (drill 0.3) (layers "F.Cu" "B.Cu") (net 18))
 (via (at 93.8 37.8) (size 0.6) (drill 0.3) (layers "F.Cu" "B.Cu") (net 18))
 (segment (start 93.8 37.8) (end 82.5 37.8) (width 0.4) (layer "B.Cu") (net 18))
 (segment (start 79.3 37.8) (end 78.9 37.4) (width 0.4) (layer "B.Cu") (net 18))
 (segment (start 82.5 37.8) (end 79.3 37.8) (width 0.4) (layer "B.Cu") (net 18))
 (segment (start 98.8 37.7) (end 98.5 37.4) (width 0.4) (layer "F.Cu") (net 14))
 (segment (start 98.2 37.1) (end 98.2 34.7) (width 0.4) (layer "F.Cu") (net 14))
 (segment (start 105.8 37.79) (end 104.31 37.79) (width 0.4) (layer "F.Cu") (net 14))
 (segment (start 88.8 33.5) (end 88.8 30.74) (width 0.4) (layer "F.Cu") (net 14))
 (segment (start 104.31 37.79) (end 104.3 37.8) (width 0.4) (layer "F.Cu") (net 14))
 (segment (start 88.8 30.74) (end 88.88 30.66) (width 0.4) (layer "F.Cu") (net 14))
 (segment (start 98.5 37.4) (end 98.2 37.1) (width 0.4) (layer "F.Cu") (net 14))
 (via (at 98.2 34.7) (size 0.6) (drill 0.3) (layers "F.Cu" "B.Cu") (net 14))
 (via (at 104.3 37.8) (size 0.6) (drill 0.3) (layers "F.Cu" "B.Cu") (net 14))
 (via (at 98.8 37.7) (size 0.6) (drill 0.3) (layers "F.Cu" "B.Cu") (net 14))
 (via (at 88.8 33.5) (size 0.6) (drill 0.3) (layers "F.Cu" "B.Cu") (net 14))
 (segment (start 94.6 33.7) (end 91 33.7) (width 0.4) (layer "B.Cu") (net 14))
 (segment (start 98.9 37.8) (end 98.8 37.7) (width 0.4) (layer "B.Cu") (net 14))
 (segment (start 89 33.7) (end 88.8 33.5) (width 0.4) (layer "B.Cu") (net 14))
 (segment (start 104.3 37.8) (end 98.9 37.8) (width 0.4) (layer "B.Cu") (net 14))
 (segment (start 91 33.7) (end 89 33.7) (width 0.4) (layer "B.Cu") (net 14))
 (segment (start 95.3 34.4) (end 94.6 33.7) (width 0.4) (layer "B.Cu") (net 14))
 (segment (start 98.2 34.7) (end 97.9 34.4) (width 0.4) (layer "B.Cu") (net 14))
 (segment (start 97.9 34.4) (end 95.3 34.4) (width 0.4) (layer "B.Cu") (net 14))
 (segment (start 93.93 42.87) (end 93.9 42.9) (width 0.4) (layer "F.Cu") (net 16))
 (segment (start 95.4 42.87) (end 93.93 42.87) (width 0.4) (layer "F.Cu") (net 16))
 (segment (start 83.8 41.1) (end 83.8 30.66) (width 0.4) (layer "F.Cu") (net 16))
 (via (at 93.9 42.9) (size 0.6) (drill 0.3) (layers "F.Cu" "B.Cu") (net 16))
 (via (at 83.8 41.1) (size 0.6) (drill 0.3) (layers "F.Cu" "B.Cu") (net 16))
 (segment (start 85.1 42.4) (end 83.8 41.1) (width 0.4) (layer "B.Cu") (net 16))
 (segment (start 93.9 42.9) (end 93 42.9) (width 0.4) (layer "B.Cu") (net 16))
 (segment (start 92.5 42.4) (end 85.1 42.4) (width 0.4) (layer "B.Cu") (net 16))
 (segment (start 93 42.9) (end 92.5 42.4) (width 0.4) (layer "B.Cu") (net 16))
 (segment (start 86.34 39.54) (end 86.34 30.66) (width 0.4) (layer "F.Cu") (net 15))
 (segment (start 86.6 39.8) (end 86.34 39.54) (width 0.4) (layer "F.Cu") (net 15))
 (segment (start 93.93 40.33) (end 93.9 40.3) (width 0.4) (layer "F.Cu") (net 15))
 (segment (start 95.4 40.33) (end 93.93 40.33) (width 0.4) (layer "F.Cu") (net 15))
 (via (at 93.9 40.3) (size 0.6) (drill 0.3) (layers "F.Cu" "B.Cu") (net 15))
 (via (at 86.6 39.8) (size 0.6) (drill 0.3) (layers "F.Cu" "B.Cu") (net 15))
 (segment (start 93.9 40.3) (end 87.1 40.3) (width 0.4) (layer "B.Cu") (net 15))
 (segment (start 87.1 40.3) (end 86.6 39.8) (width 0.4) (layer "B.Cu") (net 15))
 (segment (start 87.3 44.94) (end 86.34 45.9) (width 0.4) (layer "F.Cu") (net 10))
 (segment (start 87.3 38.01005) (end 87.3 44.94) (width 0.4) (layer "F.Cu") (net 10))
 (segment (start 95.1 29.3) (end 95.1 32.1) (width 0.4) (layer "F.Cu") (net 10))
 (segment (start 94.4 27) (end 95.1 27.7) (width 0.4) (layer "F.Cu") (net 10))
 (segment (start 90.4 31.9) (end 90.4 34.91005) (width 0.4) (layer "F.Cu") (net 10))
 (segment (start 89.68 25.5) (end 89.7 25.5) (width 0.4) (layer "F.Cu") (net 10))
 (segment (start 90.4 34.91005) (end 87.3 38.01005) (width 0.4) (layer "F.Cu") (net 10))
 (segment (start 95.1 27.7) (end 95.1 29.3) (width 0.4) (layer "F.Cu") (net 10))
 (segment (start 95.1 32.1) (end 94.9 32.3) (width 0.4) (layer "F.Cu") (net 10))
 (via (at 94.9 32.3) (size 0.6) (drill 0.3) (layers "F.Cu" "B.Cu") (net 10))
 (via (at 90.4 31.9) (size 0.6) (drill 0.3) (layers "F.Cu" "B.Cu") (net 10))
 (via (at 94.4 27) (size 0.6) (drill 0.3) (layers "F.Cu" "B.Cu") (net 10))
 (segment (start 94.15 26.75) (end 94.4 27) (width 0.4) (layer "B.Cu") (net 10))
 (segment (start 94.9 32.3) (end 90.8 32.3) (width 0.4) (layer "B.Cu") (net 10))
 (segment (start 90.8 32.3) (end 90.4 31.9) (width 0.4) (layer "B.Cu") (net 10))
 (segment (start 90.93 26.75) (end 94.15 26.75) (width 0.4) (layer "B.Cu") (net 10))
 (segment (start 89.68 25.5) (end 90.93 26.75) (width 0.4) (layer "B.Cu") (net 10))
 (segment (start 98.9 36.4) (end 98.9 26.2) (width 0.4) (layer "F.Cu") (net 11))
 (segment (start 98.9 26.2) (end 97.6 24.9) (width 0.4) (layer "F.Cu") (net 11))
 (segment (start 88.88 37.42) (end 89.4 36.9) (width 0.4) (layer "F.Cu") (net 11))
 (segment (start 88.88 45.9) (end 88.88 37.42) (width 0.4) (layer "F.Cu") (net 11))
 (via (at 97.6 24.9) (size 0.6) (drill 0.3) (layers "F.Cu" "B.Cu") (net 11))
 (via (at 89.4 36.9) (size 0.6) (drill 0.3) (layers "F.Cu" "B.Cu") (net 11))
 (via (at 98.9 36.4) (size 0.6) (drill 0.3) (layers "F.Cu" "B.Cu") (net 11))
 (segment (start 98.4 36.9) (end 98.9 36.4) (width 0.4) (layer "B.Cu") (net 11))
 (segment (start 92.82 24.9) (end 92.22 25.5) (width 0.4) (layer "B.Cu") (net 11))
 (segment (start 89.4 36.9) (end 98.4 36.9) (width 0.4) (layer "B.Cu") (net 11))
 (segment (start 97.6 24.9) (end 92.82 24.9) (width 0.4) (layer "B.Cu") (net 11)))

